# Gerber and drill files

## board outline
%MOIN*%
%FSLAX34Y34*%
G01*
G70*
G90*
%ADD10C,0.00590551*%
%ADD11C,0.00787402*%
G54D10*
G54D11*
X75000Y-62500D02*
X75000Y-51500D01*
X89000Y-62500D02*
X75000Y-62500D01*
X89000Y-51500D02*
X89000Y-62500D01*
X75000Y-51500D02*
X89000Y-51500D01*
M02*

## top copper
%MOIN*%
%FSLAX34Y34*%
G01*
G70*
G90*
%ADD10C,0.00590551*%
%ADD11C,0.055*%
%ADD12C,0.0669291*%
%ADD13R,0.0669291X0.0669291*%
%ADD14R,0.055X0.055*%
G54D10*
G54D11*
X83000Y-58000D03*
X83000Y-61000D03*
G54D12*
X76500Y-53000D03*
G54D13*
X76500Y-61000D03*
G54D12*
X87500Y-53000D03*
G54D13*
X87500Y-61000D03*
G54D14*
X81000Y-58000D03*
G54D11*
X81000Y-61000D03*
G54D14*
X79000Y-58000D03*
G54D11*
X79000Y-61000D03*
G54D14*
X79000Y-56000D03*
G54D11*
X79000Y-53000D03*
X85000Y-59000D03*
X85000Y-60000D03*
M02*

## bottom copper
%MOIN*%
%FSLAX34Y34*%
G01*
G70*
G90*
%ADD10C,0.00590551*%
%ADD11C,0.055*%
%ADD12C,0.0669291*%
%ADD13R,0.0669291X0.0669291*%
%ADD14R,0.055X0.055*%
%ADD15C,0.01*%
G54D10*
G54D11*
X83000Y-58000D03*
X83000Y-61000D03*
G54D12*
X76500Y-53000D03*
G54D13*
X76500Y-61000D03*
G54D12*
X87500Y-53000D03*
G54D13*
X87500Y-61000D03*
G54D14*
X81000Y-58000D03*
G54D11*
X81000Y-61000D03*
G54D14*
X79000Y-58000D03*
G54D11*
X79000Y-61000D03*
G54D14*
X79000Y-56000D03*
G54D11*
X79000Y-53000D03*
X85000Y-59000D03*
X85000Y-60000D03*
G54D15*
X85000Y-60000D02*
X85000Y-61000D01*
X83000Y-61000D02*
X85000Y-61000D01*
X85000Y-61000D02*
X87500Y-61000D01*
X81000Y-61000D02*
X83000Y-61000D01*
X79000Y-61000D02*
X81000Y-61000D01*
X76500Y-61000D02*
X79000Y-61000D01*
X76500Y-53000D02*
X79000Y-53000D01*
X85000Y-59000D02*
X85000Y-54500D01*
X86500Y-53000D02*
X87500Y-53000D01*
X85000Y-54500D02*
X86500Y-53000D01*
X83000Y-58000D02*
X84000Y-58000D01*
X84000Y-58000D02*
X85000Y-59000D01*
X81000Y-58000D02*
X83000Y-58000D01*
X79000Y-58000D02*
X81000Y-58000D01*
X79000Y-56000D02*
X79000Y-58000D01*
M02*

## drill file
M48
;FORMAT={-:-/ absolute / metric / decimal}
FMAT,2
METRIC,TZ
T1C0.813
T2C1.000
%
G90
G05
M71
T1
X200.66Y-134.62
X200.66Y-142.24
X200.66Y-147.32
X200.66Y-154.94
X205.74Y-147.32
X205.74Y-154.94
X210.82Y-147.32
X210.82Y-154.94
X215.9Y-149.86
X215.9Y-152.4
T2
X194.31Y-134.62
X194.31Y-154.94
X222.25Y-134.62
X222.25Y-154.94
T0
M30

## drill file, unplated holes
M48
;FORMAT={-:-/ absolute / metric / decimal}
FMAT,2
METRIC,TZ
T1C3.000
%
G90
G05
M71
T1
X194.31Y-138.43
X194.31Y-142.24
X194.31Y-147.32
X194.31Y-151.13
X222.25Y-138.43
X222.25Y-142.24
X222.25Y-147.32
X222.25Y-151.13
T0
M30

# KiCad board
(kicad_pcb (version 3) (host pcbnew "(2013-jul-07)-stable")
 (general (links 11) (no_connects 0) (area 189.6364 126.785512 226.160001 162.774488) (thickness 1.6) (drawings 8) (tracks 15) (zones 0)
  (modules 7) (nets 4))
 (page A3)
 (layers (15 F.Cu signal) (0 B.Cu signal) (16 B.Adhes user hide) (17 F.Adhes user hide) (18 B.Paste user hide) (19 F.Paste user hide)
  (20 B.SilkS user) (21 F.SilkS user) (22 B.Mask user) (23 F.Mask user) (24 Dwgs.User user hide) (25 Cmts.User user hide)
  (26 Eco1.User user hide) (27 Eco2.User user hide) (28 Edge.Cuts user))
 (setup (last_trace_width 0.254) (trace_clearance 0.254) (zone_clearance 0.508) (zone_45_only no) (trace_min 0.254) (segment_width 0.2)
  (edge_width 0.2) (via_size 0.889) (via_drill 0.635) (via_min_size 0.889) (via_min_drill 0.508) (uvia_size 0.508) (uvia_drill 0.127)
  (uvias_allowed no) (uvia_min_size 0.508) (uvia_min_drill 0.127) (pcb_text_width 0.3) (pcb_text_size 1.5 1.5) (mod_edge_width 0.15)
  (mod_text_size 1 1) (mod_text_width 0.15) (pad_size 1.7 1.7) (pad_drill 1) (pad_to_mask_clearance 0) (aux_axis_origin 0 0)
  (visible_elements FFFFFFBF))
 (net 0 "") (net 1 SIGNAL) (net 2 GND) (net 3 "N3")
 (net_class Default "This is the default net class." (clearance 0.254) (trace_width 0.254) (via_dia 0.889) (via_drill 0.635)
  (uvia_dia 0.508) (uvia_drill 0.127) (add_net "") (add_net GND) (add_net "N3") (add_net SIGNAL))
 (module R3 (layer F.Cu) (at 210.82 151.13 270) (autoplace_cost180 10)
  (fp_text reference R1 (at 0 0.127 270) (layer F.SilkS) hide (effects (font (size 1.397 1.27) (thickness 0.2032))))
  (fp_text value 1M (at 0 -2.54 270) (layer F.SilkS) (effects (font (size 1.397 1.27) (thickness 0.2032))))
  (pad 1 thru_hole circle (at -3.81 0 270) (size 1.397 1.397) (drill 0.8128) (layers *.Cu *.Mask F.SilkS) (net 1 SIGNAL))
  (pad 2 thru_hole circle (at 3.81 0 270) (size 1.397 1.397) (drill 0.8128) (layers *.Cu *.Mask F.SilkS) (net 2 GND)))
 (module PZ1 (layer F.Cu) (at 194.31 144.78 270)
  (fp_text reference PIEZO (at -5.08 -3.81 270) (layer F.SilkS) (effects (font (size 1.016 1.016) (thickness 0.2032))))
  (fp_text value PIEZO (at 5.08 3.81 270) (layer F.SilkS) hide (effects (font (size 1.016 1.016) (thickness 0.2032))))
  (pad 1 thru_hole circle (at -10.16 0 270) (size 1.7 1.7) (drill 1) (layers *.Cu *.Mask F.SilkS) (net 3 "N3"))
  (pad 2 thru_hole rect (at 10.16 0 270) (size 1.7 1.7) (drill 1) (layers *.Cu *.Mask F.SilkS) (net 2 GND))
  (pad "" np_thru_hole circle (at 6.35 0 270) (size 3 3) (drill 3) (layers *.Cu *.Mask F.SilkS))
  (pad "" np_thru_hole circle (at 2.54 0 270) (size 3 3) (drill 3) (layers *.Cu *.Mask F.SilkS))
  (pad "" np_thru_hole circle (at -2.54 0 270) (size 3 3) (drill 3) (layers *.Cu *.Mask F.SilkS))
  (pad "" np_thru_hole circle (at -6.35 0 270) (size 3 3) (drill 3) (layers *.Cu *.Mask F.SilkS)))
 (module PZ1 (layer F.Cu) (at 222.25 144.78 270)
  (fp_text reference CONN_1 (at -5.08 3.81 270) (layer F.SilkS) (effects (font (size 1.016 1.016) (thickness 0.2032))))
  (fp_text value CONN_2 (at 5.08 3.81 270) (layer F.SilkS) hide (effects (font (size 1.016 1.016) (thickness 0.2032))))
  (pad 1 thru_hole circle (at -10.16 0 270) (size 1.7 1.7) (drill 1) (layers *.Cu *.Mask F.SilkS) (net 1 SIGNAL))
  (pad 2 thru_hole rect (at 10.16 0 270) (size 1.7 1.7) (drill 1) (layers *.Cu *.Mask F.SilkS) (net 2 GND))
  (pad "" np_thru_hole circle (at 6.35 0 270) (size 3 3) (drill 3) (layers *.Cu *.Mask F.SilkS))
  (pad "" np_thru_hole circle (at 2.54 0 270) (size 3 3) (drill 3) (layers *.Cu *.Mask F.SilkS))
  (pad "" np_thru_hole circle (at -2.54 0 270) (size 3 3) (drill 3) (layers *.Cu *.Mask F.SilkS))
  (pad "" np_thru_hole circle (at -6.35 0 270) (size 3 3) (drill 3) (layers *.Cu *.Mask F.SilkS)))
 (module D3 (layer F.Cu) (at 205.74 151.13 90)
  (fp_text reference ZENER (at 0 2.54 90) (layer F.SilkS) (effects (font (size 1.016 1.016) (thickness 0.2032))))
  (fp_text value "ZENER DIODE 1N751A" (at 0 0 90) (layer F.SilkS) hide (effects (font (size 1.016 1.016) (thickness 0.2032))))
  (pad 2 thru_hole rect (at 3.81 0 90) (size 1.397 1.397) (drill 0.8128) (layers *.Cu *.Mask F.SilkS) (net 1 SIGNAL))
  (pad 1 thru_hole circle (at -3.81 0 90) (size 1.397 1.397) (drill 0.8128) (layers *.Cu *.Mask F.SilkS) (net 2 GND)))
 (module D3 (layer F.Cu) (at 200.66 151.13 90)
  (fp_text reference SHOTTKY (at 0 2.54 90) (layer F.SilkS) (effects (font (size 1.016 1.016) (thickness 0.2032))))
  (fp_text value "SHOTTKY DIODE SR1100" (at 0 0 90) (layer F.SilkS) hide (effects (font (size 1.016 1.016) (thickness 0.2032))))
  (pad 2 thru_hole rect (at 3.81 0 90) (size 1.397 1.397) (drill 0.8128) (layers *.Cu *.Mask F.SilkS) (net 1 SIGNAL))
  (pad 1 thru_hole circle (at -3.81 0 90) (size 1.397 1.397) (drill 0.8128) (layers *.Cu *.Mask F.SilkS) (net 2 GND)))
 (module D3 (layer F.Cu) (at 200.66 138.43 270)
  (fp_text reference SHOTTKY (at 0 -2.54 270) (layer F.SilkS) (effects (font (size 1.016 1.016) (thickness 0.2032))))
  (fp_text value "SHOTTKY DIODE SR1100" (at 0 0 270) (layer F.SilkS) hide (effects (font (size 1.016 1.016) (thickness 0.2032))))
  (pad 2 thru_hole rect (at 3.81 0 270) (size 1.397 1.397) (drill 0.8128) (layers *.Cu *.Mask F.SilkS) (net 1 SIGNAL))
  (pad 1 thru_hole circle (at -3.81 0 270) (size 1.397 1.397) (drill 0.8128) (layers *.Cu *.Mask F.SilkS) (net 3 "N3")))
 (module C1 (layer F.Cu) (at 215.9 151.13 270)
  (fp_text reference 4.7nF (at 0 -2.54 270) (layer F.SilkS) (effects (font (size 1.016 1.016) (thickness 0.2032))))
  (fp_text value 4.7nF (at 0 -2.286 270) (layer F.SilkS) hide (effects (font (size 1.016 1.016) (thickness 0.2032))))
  (pad 1 thru_hole circle (at -1.27 0 270) (size 1.397 1.397) (drill 0.8128) (layers *.Cu *.Mask F.SilkS) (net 1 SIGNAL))
  (pad 2 thru_hole circle (at 1.27 0 270) (size 1.397 1.397) (drill 0.8128) (layers *.Cu *.Mask F.SilkS) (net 2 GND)))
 (gr_line (start 190.5 158.75) (end 190.5 130.81) (angle 90) (layer Edge.Cuts) (width 0.2))
 (gr_line (start 226.06 158.75) (end 190.5 158.75) (angle 90) (layer Edge.Cuts) (width 0.2))
 (gr_line (start 226.06 130.81) (end 226.06 158.75) (angle 90) (layer Edge.Cuts) (width 0.2))
 (gr_line (start 190.5 130.81) (end 226.06 130.81) (angle 90) (layer Edge.Cuts) (width 0.2))
 (segment (start 215.9 152.4) (end 215.9 154.94) (width 0.254) (layer B.Cu) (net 2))
 (segment (start 210.82 154.94) (end 215.9 154.94) (width 0.254) (layer B.Cu) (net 2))
 (segment (start 215.9 154.94) (end 222.25 154.94) (width 0.254) (layer B.Cu) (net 2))
 (segment (start 205.74 154.94) (end 210.82 154.94) (width 0.254) (layer B.Cu) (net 2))
 (segment (start 200.66 154.94) (end 205.74 154.94) (width 0.254) (layer B.Cu) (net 2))
 (segment (start 194.31 154.94) (end 200.66 154.94) (width 0.254) (layer B.Cu) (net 2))
 (segment (start 194.31 134.62) (end 200.66 134.62) (width 0.254) (layer B.Cu) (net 3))
 (segment (start 215.9 149.86) (end 215.9 138.43) (width 0.254) (layer B.Cu) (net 1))
 (segment (start 219.71 134.62) (end 222.25 134.62) (width 0.254) (layer B.Cu) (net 1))
 (segment (start 215.9 138.43) (end 219.71 134.62) (width 0.254) (layer B.Cu) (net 1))
 (segment (start 210.82 147.32) (end 213.36 147.32) (width 0.254) (layer B.Cu) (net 1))
 (segment (start 213.36 147.32) (end 215.9 149.86) (width 0.254) (layer B.Cu) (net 1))
 (segment (start 205.74 147.32) (end 210.82 147.32) (width 0.254) (layer B.Cu) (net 1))
 (segment (start 200.66 147.32) (end 205.74 147.32) (width 0.254) (layer B.Cu) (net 1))
 (segment (start 200.66 142.24) (end 200.66 147.32) (width 0.254) (layer B.Cu) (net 1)))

